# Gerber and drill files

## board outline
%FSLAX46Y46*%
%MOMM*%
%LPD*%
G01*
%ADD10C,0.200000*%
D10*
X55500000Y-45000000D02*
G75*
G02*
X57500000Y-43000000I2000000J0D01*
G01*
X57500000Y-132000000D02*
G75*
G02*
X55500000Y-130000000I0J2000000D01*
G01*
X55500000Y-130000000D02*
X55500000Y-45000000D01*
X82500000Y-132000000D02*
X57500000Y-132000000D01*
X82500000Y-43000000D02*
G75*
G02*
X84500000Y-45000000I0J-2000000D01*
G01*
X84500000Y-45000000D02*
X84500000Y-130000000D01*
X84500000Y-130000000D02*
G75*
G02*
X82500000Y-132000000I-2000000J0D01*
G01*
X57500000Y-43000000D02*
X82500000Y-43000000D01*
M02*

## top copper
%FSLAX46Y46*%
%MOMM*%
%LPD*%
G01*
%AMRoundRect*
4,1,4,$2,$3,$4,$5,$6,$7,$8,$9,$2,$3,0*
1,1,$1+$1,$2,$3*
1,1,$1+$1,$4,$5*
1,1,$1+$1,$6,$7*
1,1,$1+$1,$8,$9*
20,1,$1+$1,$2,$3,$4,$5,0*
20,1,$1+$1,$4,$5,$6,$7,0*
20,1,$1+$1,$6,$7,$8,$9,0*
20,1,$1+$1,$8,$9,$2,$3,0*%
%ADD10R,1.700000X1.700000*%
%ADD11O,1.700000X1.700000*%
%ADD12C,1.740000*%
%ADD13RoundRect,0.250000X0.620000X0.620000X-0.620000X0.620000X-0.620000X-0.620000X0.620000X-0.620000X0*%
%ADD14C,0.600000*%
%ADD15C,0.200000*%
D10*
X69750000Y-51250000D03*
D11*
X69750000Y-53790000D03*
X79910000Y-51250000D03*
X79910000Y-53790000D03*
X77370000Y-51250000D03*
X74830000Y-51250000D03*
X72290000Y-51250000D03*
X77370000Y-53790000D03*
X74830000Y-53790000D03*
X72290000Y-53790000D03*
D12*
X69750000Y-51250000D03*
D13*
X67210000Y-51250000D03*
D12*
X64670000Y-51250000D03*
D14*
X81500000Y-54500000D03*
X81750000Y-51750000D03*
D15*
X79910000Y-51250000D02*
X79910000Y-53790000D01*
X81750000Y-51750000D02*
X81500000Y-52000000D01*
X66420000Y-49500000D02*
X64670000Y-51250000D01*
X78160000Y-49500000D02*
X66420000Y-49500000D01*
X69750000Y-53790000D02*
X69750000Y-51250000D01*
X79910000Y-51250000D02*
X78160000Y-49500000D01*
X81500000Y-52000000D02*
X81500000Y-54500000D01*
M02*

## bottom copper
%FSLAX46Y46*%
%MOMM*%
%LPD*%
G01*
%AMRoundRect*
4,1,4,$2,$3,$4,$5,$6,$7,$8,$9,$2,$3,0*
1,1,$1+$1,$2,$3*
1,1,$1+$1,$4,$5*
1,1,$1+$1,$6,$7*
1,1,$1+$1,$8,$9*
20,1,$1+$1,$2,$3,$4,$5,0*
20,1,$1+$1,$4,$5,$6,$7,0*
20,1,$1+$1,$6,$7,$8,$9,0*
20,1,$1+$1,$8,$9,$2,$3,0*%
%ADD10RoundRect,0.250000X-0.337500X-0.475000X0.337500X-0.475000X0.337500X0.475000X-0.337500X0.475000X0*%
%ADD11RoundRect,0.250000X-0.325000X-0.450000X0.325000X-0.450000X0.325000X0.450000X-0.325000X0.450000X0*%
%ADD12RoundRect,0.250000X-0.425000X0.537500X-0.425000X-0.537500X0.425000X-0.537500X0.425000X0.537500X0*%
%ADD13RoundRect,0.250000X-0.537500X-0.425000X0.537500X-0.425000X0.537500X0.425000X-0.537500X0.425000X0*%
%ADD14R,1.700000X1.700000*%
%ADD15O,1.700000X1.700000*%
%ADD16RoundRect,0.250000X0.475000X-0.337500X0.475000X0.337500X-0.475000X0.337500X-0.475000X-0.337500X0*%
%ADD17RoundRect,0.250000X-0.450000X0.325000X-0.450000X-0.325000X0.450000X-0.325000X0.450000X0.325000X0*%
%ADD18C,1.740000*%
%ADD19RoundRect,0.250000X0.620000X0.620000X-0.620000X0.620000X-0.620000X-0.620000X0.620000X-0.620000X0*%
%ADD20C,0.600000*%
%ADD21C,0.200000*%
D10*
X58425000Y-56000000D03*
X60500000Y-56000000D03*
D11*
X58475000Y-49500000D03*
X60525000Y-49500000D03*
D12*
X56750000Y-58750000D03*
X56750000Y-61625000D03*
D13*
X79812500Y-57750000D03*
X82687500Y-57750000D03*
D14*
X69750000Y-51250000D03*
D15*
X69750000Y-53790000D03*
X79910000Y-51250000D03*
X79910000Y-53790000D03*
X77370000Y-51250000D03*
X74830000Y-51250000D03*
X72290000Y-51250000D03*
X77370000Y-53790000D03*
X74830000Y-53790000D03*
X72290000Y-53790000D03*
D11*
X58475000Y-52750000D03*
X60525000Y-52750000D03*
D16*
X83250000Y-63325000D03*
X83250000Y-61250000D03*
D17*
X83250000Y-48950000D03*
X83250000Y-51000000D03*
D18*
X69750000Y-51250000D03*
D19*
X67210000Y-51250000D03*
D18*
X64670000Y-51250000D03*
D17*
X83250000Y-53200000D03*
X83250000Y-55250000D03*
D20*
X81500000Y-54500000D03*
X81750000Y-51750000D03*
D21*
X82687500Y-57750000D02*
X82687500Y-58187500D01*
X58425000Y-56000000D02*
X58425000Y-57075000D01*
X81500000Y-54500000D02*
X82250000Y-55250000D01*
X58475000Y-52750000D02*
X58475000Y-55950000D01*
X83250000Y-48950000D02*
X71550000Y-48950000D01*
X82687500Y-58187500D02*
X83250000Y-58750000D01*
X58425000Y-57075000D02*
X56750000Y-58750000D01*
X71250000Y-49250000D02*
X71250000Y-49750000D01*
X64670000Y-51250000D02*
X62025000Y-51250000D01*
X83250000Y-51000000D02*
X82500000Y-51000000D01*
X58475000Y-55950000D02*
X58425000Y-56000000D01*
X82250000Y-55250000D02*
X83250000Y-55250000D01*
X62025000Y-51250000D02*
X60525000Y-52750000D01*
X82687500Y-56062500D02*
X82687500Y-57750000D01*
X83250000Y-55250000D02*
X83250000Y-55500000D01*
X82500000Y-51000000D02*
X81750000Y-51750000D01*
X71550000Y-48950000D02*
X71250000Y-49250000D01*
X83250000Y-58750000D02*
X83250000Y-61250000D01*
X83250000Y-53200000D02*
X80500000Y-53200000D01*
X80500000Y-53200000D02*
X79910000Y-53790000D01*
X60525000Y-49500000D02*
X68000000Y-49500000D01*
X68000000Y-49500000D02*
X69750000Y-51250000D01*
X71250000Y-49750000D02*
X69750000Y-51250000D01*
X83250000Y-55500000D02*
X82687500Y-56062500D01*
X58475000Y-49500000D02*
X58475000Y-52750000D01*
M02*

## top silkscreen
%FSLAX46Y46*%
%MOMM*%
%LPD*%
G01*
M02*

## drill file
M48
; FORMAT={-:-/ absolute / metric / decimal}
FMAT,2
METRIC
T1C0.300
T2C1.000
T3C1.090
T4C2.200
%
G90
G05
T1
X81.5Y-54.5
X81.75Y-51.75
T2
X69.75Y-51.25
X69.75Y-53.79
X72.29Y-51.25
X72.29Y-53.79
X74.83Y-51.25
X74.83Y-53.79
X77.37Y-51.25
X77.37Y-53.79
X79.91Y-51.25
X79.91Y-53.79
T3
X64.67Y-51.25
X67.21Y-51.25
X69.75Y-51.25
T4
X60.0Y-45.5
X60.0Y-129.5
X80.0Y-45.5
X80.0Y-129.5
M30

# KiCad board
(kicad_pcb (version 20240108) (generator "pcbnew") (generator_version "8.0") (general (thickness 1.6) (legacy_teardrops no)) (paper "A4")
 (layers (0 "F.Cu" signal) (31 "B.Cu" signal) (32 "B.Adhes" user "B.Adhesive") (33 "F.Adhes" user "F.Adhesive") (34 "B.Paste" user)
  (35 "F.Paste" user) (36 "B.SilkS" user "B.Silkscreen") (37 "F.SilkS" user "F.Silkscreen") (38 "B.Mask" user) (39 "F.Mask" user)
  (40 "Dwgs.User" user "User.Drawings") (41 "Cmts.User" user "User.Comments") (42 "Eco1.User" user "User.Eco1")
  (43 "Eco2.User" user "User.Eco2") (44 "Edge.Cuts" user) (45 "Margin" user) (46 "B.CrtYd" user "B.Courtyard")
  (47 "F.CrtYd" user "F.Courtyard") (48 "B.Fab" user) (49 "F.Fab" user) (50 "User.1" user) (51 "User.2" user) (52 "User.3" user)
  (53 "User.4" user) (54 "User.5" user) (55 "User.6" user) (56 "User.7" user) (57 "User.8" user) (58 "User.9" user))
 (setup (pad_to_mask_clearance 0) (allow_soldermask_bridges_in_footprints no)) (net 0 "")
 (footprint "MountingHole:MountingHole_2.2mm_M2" (layer "F.Cu") (at 80 45.5)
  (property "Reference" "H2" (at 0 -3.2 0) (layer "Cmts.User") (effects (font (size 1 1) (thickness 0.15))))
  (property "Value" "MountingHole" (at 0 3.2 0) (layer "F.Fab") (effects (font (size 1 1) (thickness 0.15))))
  (pad "" np_thru_hole circle (at 0 0) (size 2.2 2.2) (drill 2.2) (layers "F&B.Cu" "*.Mask")))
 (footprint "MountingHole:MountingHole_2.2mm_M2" (layer "F.Cu") (at 60 129.5)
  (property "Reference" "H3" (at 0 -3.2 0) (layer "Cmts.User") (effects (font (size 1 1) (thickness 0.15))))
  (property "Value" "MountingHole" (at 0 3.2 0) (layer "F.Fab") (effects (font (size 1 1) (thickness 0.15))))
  (pad "" np_thru_hole circle (at 0 0) (size 2.2 2.2) (drill 2.2) (layers "F&B.Cu" "*.Mask")))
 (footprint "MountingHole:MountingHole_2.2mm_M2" (layer "F.Cu") (at 60 45.5)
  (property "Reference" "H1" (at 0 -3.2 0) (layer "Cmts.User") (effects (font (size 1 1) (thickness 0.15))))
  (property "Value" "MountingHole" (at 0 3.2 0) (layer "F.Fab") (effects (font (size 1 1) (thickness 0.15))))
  (pad "" np_thru_hole circle (at 0 0) (size 2.2 2.2) (drill 2.2) (layers "F&B.Cu" "*.Mask")))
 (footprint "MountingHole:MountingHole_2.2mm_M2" (layer "F.Cu") (at 80 129.5)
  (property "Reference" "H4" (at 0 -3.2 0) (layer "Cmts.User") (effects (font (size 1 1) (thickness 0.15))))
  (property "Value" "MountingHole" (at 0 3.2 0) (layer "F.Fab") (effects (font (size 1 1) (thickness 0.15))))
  (pad "" np_thru_hole circle (at 0 0) (size 2.2 2.2) (drill 2.2) (layers "F&B.Cu" "*.Mask")))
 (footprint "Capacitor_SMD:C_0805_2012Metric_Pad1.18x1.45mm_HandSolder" (layer "B.Cu") (at 59.4625 56)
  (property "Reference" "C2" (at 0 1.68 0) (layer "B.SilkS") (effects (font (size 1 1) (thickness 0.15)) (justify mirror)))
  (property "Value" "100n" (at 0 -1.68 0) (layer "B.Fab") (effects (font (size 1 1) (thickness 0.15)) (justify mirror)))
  (pad "1" smd roundrect (at -1.0375 0) (size 1.175 1.45) (layers "B.Cu" "B.Paste" "B.Mask") (roundrect_rratio 0.212766))
  (pad "2" smd roundrect (at 1.0375 0) (size 1.175 1.45) (layers "B.Cu" "B.Paste" "B.Mask") (roundrect_rratio 0.212766)))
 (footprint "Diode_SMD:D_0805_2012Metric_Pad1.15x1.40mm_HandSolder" (layer "B.Cu") (at 59.5 49.5)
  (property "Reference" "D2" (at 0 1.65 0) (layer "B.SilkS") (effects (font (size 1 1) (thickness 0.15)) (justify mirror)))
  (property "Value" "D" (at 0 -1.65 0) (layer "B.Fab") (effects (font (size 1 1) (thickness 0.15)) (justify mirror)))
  (pad "1" smd roundrect (at -1.025 0) (size 1.15 1.4) (layers "B.Cu" "B.Paste" "B.Mask") (roundrect_rratio 0.217391))
  (pad "2" smd roundrect (at 1.025 0) (size 1.15 1.4) (layers "B.Cu" "B.Paste" "B.Mask") (roundrect_rratio 0.217391)))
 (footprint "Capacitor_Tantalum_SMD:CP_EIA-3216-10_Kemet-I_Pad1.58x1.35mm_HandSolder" (layer "B.Cu") (at 56.75 60.1875 -90)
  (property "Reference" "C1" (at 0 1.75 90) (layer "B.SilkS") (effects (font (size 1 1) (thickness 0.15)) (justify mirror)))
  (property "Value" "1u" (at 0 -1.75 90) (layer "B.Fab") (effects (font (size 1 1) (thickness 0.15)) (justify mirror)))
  (pad "1" smd roundrect (at -1.4375 0 270) (size 1.575 1.35) (layers "B.Cu" "B.Paste" "B.Mask") (roundrect_rratio 0.185185))
  (pad "2" smd roundrect (at 1.4375 0 270) (size 1.575 1.35) (layers "B.Cu" "B.Paste" "B.Mask") (roundrect_rratio 0.185185)))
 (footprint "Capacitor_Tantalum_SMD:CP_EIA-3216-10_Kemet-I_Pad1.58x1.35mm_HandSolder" (layer "B.Cu") (at 81.25 57.75)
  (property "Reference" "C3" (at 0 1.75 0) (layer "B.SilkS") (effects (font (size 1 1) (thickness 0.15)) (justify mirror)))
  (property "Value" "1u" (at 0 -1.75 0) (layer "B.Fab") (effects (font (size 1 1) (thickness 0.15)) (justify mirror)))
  (pad "1" smd roundrect (at -1.4375 0) (size 1.575 1.35) (layers "B.Cu" "B.Paste" "B.Mask") (roundrect_rratio 0.185185))
  (pad "2" smd roundrect (at 1.4375 0) (size 1.575 1.35) (layers "B.Cu" "B.Paste" "B.Mask") (roundrect_rratio 0.185185)))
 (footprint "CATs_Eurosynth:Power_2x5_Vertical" (layer "B.Cu") (at 69.75 51.25 -90)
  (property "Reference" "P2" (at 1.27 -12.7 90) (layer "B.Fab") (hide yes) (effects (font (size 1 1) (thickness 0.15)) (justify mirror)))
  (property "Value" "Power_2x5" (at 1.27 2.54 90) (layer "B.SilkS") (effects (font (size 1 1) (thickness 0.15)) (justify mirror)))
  (pad "+12V" thru_hole rect (at 0 0 270) (size 1.7 1.7) (drill 1) (layers "*.Cu" "*.Mask") (remove_unused_layers no))
  (pad "+12V" thru_hole oval (at 2.54 0 270) (size 1.7 1.7) (drill 1) (layers "*.Cu" "*.Mask") (remove_unused_layers no))
  (pad "-12V" thru_hole oval (at 0 -10.16 270) (size 1.7 1.7) (drill 1) (layers "*.Cu" "*.Mask") (remove_unused_layers no))
  (pad "-12V" thru_hole oval (at 2.54 -10.16 270) (size 1.7 1.7) (drill 1) (layers "*.Cu" "*.Mask") (remove_unused_layers no))
  (pad "GND" thru_hole oval (at 0 -7.62 270) (size 1.7 1.7) (drill 1) (layers "*.Cu" "*.Mask") (remove_unused_layers no))
  (pad "GND" thru_hole oval (at 0 -5.08 270) (size 1.7 1.7) (drill 1) (layers "*.Cu" "*.Mask") (remove_unused_layers no))
  (pad "GND" thru_hole oval (at 0 -2.54 270) (size 1.7 1.7) (drill 1) (layers "*.Cu" "*.Mask") (remove_unused_layers no))
  (pad "GND" thru_hole oval (at 2.54 -7.62 270) (size 1.7 1.7) (drill 1) (layers "*.Cu" "*.Mask") (remove_unused_layers no))
  (pad "GND" thru_hole oval (at 2.54 -5.08 270) (size 1.7 1.7) (drill 1) (layers "*.Cu" "*.Mask") (remove_unused_layers no))
  (pad "GND" thru_hole oval (at 2.54 -2.54 270) (size 1.7 1.7) (drill 1) (layers "*.Cu" "*.Mask") (remove_unused_layers no)))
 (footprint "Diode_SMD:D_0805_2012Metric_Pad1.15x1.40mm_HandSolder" (layer "B.Cu") (at 59.5 52.75)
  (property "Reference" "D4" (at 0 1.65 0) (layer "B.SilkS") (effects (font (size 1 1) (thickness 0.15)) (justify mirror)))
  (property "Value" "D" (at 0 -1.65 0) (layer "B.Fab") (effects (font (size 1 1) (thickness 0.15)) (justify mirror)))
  (pad "1" smd roundrect (at -1.025 0) (size 1.15 1.4) (layers "B.Cu" "B.Paste" "B.Mask") (roundrect_rratio 0.217391))
  (pad "2" smd roundrect (at 1.025 0) (size 1.15 1.4) (layers "B.Cu" "B.Paste" "B.Mask") (roundrect_rratio 0.217391)))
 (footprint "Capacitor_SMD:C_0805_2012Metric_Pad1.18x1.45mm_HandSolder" (layer "B.Cu") (at 83.25 62.2875 90)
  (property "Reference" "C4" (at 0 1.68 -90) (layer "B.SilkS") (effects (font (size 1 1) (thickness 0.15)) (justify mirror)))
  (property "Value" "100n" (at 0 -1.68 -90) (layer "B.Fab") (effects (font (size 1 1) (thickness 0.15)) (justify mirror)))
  (pad "1" smd roundrect (at -1.0375 0 90) (size 1.175 1.45) (layers "B.Cu" "B.Paste" "B.Mask") (roundrect_rratio 0.212766))
  (pad "2" smd roundrect (at 1.0375 0 90) (size 1.175 1.45) (layers "B.Cu" "B.Paste" "B.Mask") (roundrect_rratio 0.212766)))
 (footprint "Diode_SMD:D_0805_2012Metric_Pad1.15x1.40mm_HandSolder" (layer "B.Cu") (at 83.25 49.975 -90)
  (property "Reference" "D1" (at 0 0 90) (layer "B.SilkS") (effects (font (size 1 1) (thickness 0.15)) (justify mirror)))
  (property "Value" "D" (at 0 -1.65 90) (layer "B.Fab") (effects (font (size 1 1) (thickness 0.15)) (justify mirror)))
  (pad "1" smd roundrect (at -1.025 0 270) (size 1.15 1.4) (layers "B.Cu" "B.Paste" "B.Mask") (roundrect_rratio 0.217391))
  (pad "2" smd roundrect (at 1.025 0 270) (size 1.15 1.4) (layers "B.Cu" "B.Paste" "B.Mask") (roundrect_rratio 0.217391)))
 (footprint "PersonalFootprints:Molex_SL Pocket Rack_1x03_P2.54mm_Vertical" (layer "B.Cu") (at 69.75 51.25 180)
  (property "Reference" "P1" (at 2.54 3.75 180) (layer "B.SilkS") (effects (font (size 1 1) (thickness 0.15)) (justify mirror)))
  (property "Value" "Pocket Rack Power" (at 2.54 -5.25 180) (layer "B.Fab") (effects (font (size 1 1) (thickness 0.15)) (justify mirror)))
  (pad "1" thru_hole circle (at 0 0 180) (size 1.74 1.74) (drill 1.09) (layers "*.Cu" "*.Mask") (remove_unused_layers no))
  (pad "2" thru_hole roundrect (at 2.54 0 180) (size 1.74 1.74) (drill 1.09) (layers "*.Cu" "*.Mask") (remove_unused_layers no)
   (roundrect_rratio 0.1436781609))
  (pad "3" thru_hole circle (at 5.08 0 180) (size 1.74 1.74) (drill 1.09) (layers "*.Cu" "*.Mask") (remove_unused_layers no)))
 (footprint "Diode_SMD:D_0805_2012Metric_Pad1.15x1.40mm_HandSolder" (layer "B.Cu") (at 83.25 54.225 -90)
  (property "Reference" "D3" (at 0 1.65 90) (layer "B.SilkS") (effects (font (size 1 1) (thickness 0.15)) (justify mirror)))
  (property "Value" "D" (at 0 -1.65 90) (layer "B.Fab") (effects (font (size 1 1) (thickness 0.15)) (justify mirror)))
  (pad "1" smd roundrect (at -1.025 0 270) (size 1.15 1.4) (layers "B.Cu" "B.Paste" "B.Mask") (roundrect_rratio 0.217391))
  (pad "2" smd roundrect (at 1.025 0 270) (size 1.15 1.4) (layers "B.Cu" "B.Paste" "B.Mask") (roundrect_rratio 0.217391)))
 (gr_arc (start 55.5 45) (mid 56.085786 43.585786) (end 57.5 43) (stroke (width 0.2) (type default)) (layer "Edge.Cuts"))
 (gr_arc (start 57.5 132) (mid 56.085786 131.414214) (end 55.5 130) (stroke (width 0.2) (type default)) (layer "Edge.Cuts"))
 (gr_line (start 55.5 130) (end 55.5 45) (stroke (width 0.2) (type default)) (layer "Edge.Cuts"))
 (gr_line (start 82.5 132) (end 57.5 132) (stroke (width 0.2) (type default)) (layer "Edge.Cuts"))
 (gr_arc (start 82.5 43) (mid 83.914214 43.585786) (end 84.5 45) (stroke (width 0.2) (type default)) (layer "Edge.Cuts"))
 (gr_line (start 84.5 45) (end 84.5 130) (stroke (width 0.2) (type default)) (layer "Edge.Cuts"))
 (gr_arc (start 84.5 130) (mid 83.914214 131.414214) (end 82.5 132) (stroke (width 0.2) (type default)) (layer "Edge.Cuts"))
 (gr_line (start 57.5 43) (end 82.5 43) (stroke (width 0.2) (type default)) (layer "Edge.Cuts"))
 (segment (start 79.91 51.25) (end 79.91 53.79) (width 0.2) (layer "F.Cu") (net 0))
 (segment (start 81.75 51.75) (end 81.5 52) (width 0.2) (layer "F.Cu") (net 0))
 (segment (start 66.42 49.5) (end 64.67 51.25) (width 0.2) (layer "F.Cu") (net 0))
 (segment (start 78.16 49.5) (end 66.42 49.5) (width 0.2) (layer "F.Cu") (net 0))
 (segment (start 69.75 53.79) (end 69.75 51.25) (width 0.2) (layer "F.Cu") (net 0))
 (segment (start 79.91 51.25) (end 78.16 49.5) (width 0.2) (layer "F.Cu") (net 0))
 (segment (start 81.5 52) (end 81.5 54.5) (width 0.2) (layer "F.Cu") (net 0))
 (via (at 81.5 54.5) (size 0.6) (drill 0.3) (layers "F.Cu" "B.Cu") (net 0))
 (via (at 81.75 51.75) (size 0.6) (drill 0.3) (layers "F.Cu" "B.Cu") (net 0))
 (segment (start 82.6875 57.75) (end 82.6875 58.1875) (width 0.2) (layer "B.Cu") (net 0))
 (segment (start 58.425 56) (end 58.425 57.075) (width 0.2) (layer "B.Cu") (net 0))
 (segment (start 81.5 54.5) (end 82.25 55.25) (width 0.2) (layer "B.Cu") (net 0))
 (segment (start 58.475 52.75) (end 58.475 55.95) (width 0.2) (layer "B.Cu") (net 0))
 (segment (start 83.25 48.95) (end 71.55 48.95) (width 0.2) (layer "B.Cu") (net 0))
 (segment (start 82.6875 58.1875) (end 83.25 58.75) (width 0.2) (layer "B.Cu") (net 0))
 (segment (start 58.425 57.075) (end 56.75 58.75) (width 0.2) (layer "B.Cu") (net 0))
 (segment (start 71.25 49.25) (end 71.25 49.75) (width 0.2) (layer "B.Cu") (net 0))
 (segment (start 64.67 51.25) (end 62.025 51.25) (width 0.2) (layer "B.Cu") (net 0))
 (segment (start 83.25 51) (end 82.5 51) (width 0.2) (layer "B.Cu") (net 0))
 (segment (start 58.475 55.95) (end 58.425 56) (width 0.2) (layer "B.Cu") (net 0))
 (segment (start 82.25 55.25) (end 83.25 55.25) (width 0.2) (layer "B.Cu") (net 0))
 (segment (start 62.025 51.25) (end 60.525 52.75) (width 0.2) (layer "B.Cu") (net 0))
 (segment (start 82.6875 56.0625) (end 82.6875 57.75) (width 0.2) (layer "B.Cu") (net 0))
 (segment (start 83.25 55.25) (end 83.25 55.5) (width 0.2) (layer "B.Cu") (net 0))
 (segment (start 82.5 51) (end 81.75 51.75) (width 0.2) (layer "B.Cu") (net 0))
 (segment (start 71.55 48.95) (end 71.25 49.25) (width 0.2) (layer "B.Cu") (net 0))
 (segment (start 83.25 58.75) (end 83.25 61.25) (width 0.2) (layer "B.Cu") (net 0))
 (segment (start 83.25 53.2) (end 80.5 53.2) (width 0.2) (layer "B.Cu") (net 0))
 (segment (start 80.5 53.2) (end 79.91 53.79) (width 0.2) (layer "B.Cu") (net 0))
 (segment (start 60.525 49.5) (end 68 49.5) (width 0.2) (layer "B.Cu") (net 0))
 (segment (start 68 49.5) (end 69.75 51.25) (width 0.2) (layer "B.Cu") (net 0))
 (segment (start 71.25 49.75) (end 69.75 51.25) (width 0.2) (layer "B.Cu") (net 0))
 (segment (start 83.25 55.5) (end 82.6875 56.0625) (width 0.2) (layer "B.Cu") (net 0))
 (segment (start 58.475 49.5) (end 58.475 52.75) (width 0.2) (layer "B.Cu") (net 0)))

